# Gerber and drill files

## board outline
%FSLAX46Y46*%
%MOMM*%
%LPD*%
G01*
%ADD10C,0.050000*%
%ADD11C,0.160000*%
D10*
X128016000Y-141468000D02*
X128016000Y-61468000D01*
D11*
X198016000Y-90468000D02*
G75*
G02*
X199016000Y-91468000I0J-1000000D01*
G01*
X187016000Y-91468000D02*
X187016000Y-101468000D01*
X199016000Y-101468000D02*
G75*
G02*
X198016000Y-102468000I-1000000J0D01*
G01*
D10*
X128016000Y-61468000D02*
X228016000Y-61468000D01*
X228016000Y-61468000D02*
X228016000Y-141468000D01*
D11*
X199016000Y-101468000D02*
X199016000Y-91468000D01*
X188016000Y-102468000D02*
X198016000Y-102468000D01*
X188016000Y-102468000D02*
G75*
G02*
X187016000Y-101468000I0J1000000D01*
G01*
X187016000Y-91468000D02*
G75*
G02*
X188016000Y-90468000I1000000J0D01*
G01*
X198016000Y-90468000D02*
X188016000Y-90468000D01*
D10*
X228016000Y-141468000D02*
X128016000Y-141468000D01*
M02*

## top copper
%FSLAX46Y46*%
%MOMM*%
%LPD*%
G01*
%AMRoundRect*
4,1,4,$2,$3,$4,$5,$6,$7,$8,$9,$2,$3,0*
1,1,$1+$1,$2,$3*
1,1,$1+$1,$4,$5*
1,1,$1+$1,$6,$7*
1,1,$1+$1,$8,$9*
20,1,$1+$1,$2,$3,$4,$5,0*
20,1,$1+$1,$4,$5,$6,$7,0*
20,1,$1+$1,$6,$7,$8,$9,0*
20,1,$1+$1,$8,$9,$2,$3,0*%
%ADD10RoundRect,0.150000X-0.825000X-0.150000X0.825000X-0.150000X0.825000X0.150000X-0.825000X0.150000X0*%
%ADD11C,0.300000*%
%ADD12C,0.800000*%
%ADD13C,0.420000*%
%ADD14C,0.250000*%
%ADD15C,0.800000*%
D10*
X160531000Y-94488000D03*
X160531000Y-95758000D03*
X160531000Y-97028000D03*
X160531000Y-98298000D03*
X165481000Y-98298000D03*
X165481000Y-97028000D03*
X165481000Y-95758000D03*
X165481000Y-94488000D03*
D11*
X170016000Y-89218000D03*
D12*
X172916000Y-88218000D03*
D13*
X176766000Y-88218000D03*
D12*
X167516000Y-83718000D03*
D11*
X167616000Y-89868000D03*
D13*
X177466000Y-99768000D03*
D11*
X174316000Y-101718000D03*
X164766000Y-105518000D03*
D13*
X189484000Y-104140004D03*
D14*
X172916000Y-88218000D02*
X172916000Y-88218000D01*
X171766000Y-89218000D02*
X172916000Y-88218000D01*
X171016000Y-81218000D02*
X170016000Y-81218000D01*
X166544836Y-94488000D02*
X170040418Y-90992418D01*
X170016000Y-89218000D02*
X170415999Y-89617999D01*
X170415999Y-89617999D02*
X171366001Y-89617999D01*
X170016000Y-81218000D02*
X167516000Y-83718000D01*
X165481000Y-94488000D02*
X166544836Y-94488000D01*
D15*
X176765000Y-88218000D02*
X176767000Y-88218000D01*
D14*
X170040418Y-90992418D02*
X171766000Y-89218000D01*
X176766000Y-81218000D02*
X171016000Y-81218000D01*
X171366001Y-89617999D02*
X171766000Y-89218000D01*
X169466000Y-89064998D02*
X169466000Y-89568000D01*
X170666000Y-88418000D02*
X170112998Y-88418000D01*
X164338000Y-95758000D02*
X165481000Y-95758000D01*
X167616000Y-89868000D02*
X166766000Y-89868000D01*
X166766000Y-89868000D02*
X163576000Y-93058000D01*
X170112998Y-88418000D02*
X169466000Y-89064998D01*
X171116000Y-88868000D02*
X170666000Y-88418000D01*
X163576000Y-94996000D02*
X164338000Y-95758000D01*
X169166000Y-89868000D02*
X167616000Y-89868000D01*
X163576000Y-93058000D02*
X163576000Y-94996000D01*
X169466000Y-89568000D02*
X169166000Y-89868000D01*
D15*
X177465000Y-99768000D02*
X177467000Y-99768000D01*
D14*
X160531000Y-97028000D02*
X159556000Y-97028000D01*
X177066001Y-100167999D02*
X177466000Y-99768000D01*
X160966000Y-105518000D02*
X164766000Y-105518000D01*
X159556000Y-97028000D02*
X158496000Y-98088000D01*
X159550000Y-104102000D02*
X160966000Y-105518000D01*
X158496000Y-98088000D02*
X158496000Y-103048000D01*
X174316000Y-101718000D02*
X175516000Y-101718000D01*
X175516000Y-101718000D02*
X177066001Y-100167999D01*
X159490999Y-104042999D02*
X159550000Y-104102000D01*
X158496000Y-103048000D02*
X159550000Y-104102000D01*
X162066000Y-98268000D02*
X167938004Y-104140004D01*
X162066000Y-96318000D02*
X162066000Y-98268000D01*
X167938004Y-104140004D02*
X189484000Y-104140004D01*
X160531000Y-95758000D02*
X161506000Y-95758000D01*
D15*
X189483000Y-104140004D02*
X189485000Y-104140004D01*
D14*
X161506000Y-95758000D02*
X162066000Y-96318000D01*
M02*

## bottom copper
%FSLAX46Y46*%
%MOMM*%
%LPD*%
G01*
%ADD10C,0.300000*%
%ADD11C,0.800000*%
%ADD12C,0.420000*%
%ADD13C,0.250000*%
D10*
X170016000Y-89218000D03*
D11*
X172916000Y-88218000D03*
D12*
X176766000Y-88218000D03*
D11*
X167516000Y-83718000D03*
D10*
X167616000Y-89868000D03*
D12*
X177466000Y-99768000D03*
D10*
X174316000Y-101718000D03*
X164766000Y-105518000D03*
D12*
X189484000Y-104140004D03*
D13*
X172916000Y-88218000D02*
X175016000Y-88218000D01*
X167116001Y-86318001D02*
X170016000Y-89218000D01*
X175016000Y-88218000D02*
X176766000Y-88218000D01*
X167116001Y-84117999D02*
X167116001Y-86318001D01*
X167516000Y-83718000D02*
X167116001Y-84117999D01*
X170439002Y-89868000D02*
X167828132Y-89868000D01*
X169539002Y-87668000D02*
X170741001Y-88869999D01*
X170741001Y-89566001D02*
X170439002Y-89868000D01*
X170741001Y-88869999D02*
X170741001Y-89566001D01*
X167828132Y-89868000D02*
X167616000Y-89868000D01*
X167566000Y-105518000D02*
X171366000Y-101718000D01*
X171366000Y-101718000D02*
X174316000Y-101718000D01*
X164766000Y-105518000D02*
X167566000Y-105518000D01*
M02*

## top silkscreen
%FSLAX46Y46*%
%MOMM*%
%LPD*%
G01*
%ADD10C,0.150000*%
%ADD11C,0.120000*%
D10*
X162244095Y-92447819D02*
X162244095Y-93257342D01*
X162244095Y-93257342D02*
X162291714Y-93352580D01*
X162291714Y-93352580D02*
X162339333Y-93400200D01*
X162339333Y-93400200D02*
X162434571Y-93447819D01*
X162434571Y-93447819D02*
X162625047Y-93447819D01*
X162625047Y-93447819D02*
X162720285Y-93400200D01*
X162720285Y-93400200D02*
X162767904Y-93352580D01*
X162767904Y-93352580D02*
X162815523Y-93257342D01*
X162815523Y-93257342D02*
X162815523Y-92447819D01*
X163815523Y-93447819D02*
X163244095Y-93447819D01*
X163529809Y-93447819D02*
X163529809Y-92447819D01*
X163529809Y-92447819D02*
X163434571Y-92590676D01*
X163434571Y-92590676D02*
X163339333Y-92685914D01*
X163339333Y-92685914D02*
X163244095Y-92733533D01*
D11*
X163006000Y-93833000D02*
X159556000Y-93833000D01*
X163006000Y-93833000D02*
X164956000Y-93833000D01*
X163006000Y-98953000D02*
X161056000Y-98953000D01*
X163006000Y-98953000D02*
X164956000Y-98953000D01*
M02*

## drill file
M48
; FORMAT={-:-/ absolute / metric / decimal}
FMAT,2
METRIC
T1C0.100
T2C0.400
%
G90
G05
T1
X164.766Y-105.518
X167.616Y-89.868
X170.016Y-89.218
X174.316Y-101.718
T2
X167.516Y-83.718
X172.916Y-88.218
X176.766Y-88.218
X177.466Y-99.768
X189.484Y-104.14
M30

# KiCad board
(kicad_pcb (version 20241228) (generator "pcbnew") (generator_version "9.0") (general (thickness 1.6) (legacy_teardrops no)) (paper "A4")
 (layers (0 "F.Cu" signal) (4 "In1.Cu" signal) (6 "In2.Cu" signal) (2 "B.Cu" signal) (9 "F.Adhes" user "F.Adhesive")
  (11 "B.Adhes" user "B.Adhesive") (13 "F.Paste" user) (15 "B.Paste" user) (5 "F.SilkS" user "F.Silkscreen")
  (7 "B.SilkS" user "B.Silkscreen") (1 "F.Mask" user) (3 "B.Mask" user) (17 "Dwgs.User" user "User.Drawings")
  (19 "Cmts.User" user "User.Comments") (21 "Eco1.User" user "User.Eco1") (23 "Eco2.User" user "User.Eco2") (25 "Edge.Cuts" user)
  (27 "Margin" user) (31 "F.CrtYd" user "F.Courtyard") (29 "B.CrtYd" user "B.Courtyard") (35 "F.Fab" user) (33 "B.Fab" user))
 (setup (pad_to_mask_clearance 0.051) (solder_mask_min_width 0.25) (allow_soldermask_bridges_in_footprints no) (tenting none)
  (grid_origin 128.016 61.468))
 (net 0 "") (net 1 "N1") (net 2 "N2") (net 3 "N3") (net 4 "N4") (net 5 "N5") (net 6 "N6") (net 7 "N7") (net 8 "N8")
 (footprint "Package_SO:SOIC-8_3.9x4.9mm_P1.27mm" (layer "F.Cu") (at 163.006 96.393)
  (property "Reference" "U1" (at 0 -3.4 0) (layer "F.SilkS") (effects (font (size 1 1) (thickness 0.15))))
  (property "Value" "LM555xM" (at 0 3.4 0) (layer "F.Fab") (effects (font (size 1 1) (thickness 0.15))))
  (fp_line (start 0 -2.56) (end -3.45 -2.56) (stroke (width 0.12) (type solid)) (layer "F.SilkS"))
  (fp_line (start 0 -2.56) (end 1.95 -2.56) (stroke (width 0.12) (type solid)) (layer "F.SilkS"))
  (fp_line (start 0 2.56) (end -1.95 2.56) (stroke (width 0.12) (type solid)) (layer "F.SilkS"))
  (fp_line (start 0 2.56) (end 1.95 2.56) (stroke (width 0.12) (type solid)) (layer "F.SilkS"))
  (pad "1" smd roundrect (at -2.475 -1.905) (size 1.95 0.6) (layers "F.Cu" "F.Mask" "F.Paste") (roundrect_rratio 0.25) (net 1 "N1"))
  (pad "2" smd roundrect (at -2.475 -0.635) (size 1.95 0.6) (layers "F.Cu" "F.Mask" "F.Paste") (roundrect_rratio 0.25) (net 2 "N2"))
  (pad "3" smd roundrect (at -2.475 0.635) (size 1.95 0.6) (layers "F.Cu" "F.Mask" "F.Paste") (roundrect_rratio 0.25) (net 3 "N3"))
  (pad "4" smd roundrect (at -2.475 1.905) (size 1.95 0.6) (layers "F.Cu" "F.Mask" "F.Paste") (roundrect_rratio 0.25) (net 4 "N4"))
  (pad "5" smd roundrect (at 2.475 1.905) (size 1.95 0.6) (layers "F.Cu" "F.Mask" "F.Paste") (roundrect_rratio 0.25) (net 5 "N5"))
  (pad "6" smd roundrect (at 2.475 0.635) (size 1.95 0.6) (layers "F.Cu" "F.Mask" "F.Paste") (roundrect_rratio 0.25) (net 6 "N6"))
  (pad "7" smd roundrect (at 2.475 -0.635) (size 1.95 0.6) (layers "F.Cu" "F.Mask" "F.Paste") (roundrect_rratio 0.25) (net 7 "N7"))
  (pad "8" smd roundrect (at 2.475 -1.905) (size 1.95 0.6) (layers "F.Cu" "F.Mask" "F.Paste") (roundrect_rratio 0.25) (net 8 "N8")))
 (gr_line (start 128.016 141.468) (end 128.016 61.468) (stroke (width 0.05) (type solid)) (layer "Edge.Cuts"))
 (gr_arc (start 198.016 90.468) (mid 198.723107 90.760893) (end 199.016 91.468) (stroke (width 0.16) (type solid)) (layer "Edge.Cuts"))
 (gr_line (start 187.016 91.468) (end 187.016 101.468) (stroke (width 0.16) (type solid)) (layer "Edge.Cuts"))
 (gr_arc (start 199.016 101.468) (mid 198.723107 102.175107) (end 198.016 102.468) (stroke (width 0.16) (type solid)) (layer "Edge.Cuts"))
 (gr_line (start 128.016 61.468) (end 228.016 61.468) (stroke (width 0.05) (type solid)) (layer "Edge.Cuts"))
 (gr_line (start 228.016 61.468) (end 228.016 141.468) (stroke (width 0.05) (type solid)) (layer "Edge.Cuts"))
 (gr_line (start 199.016 101.468) (end 199.016 91.468) (stroke (width 0.16) (type solid)) (layer "Edge.Cuts"))
 (gr_line (start 188.016 102.468) (end 198.016 102.468) (stroke (width 0.16) (type solid)) (layer "Edge.Cuts"))
 (gr_arc (start 188.016 102.468) (mid 187.308893 102.175107) (end 187.016 101.468) (stroke (width 0.16) (type solid)) (layer "Edge.Cuts"))
 (gr_arc (start 187.016 91.468) (mid 187.308893 90.760893) (end 188.016 90.468) (stroke (width 0.16) (type solid)) (layer "Edge.Cuts"))
 (gr_line (start 198.016 90.468) (end 188.016 90.468) (stroke (width 0.16) (type solid)) (layer "Edge.Cuts"))
 (gr_line (start 228.016 141.468) (end 128.016 141.468) (stroke (width 0.05) (type solid)) (layer "Edge.Cuts"))
 (segment (start 172.916 88.218) (end 172.916 88.218) (width 0.25) (layer "F.Cu") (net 8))
 (segment (start 171.766 89.218) (end 172.916 88.218) (width 0.25) (layer "F.Cu") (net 8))
 (segment (start 171.016 81.218) (end 170.016 81.218) (width 0.25) (layer "F.Cu") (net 8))
 (segment (start 166.544836 94.488) (end 170.040418 90.992418) (width 0.25) (layer "F.Cu") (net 8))
 (segment (start 170.016 89.218) (end 170.415999 89.617999) (width 0.25) (layer "F.Cu") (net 8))
 (segment (start 170.415999 89.617999) (end 171.366001 89.617999) (width 0.25) (layer "F.Cu") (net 8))
 (segment (start 170.016 81.218) (end 167.516 83.718) (width 0.25) (layer "F.Cu") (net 8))
 (segment (start 165.481 94.488) (end 166.544836 94.488) (width 0.25) (layer "F.Cu") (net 8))
 (segment (start 176.765 88.218) (end 176.767 88.218) (width 0.8) (layer "F.Cu") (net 8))
 (segment (start 170.040418 90.992418) (end 171.766 89.218) (width 0.25) (layer "F.Cu") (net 8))
 (segment (start 176.766 81.218) (end 171.016 81.218) (width 0.25) (layer "F.Cu") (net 8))
 (segment (start 171.366001 89.617999) (end 171.766 89.218) (width 0.25) (layer "F.Cu") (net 8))
 (via (at 170.016 89.218) (size 0.3) (drill 0.1) (layers "F.Cu" "B.Cu") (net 8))
 (via (at 172.916 88.218) (size 0.8) (drill 0.4) (layers "F.Cu" "B.Cu") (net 8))
 (via (at 176.766 88.218) (size 0.42) (drill 0.4) (layers "F.Cu" "B.Cu") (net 8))
 (via (at 167.516 83.718) (size 0.8) (drill 0.4) (layers "F.Cu" "B.Cu") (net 8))
 (segment (start 172.916 88.218) (end 175.016 88.218) (width 0.25) (layer "B.Cu") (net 8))
 (segment (start 167.116001 86.318001) (end 170.016 89.218) (width 0.25) (layer "B.Cu") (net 8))
 (segment (start 175.016 88.218) (end 176.766 88.218) (width 0.25) (layer "B.Cu") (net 8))
 (segment (start 167.116001 84.117999) (end 167.116001 86.318001) (width 0.25) (layer "B.Cu") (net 8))
 (segment (start 167.516 83.718) (end 167.116001 84.117999) (width 0.25) (layer "B.Cu") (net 8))
 (segment (start 169.466 89.064998) (end 169.466 89.568) (width 0.25) (layer "F.Cu") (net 7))
 (segment (start 170.666 88.418) (end 170.112998 88.418) (width 0.25) (layer "F.Cu") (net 7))
 (segment (start 164.338 95.758) (end 165.481 95.758) (width 0.25) (layer "F.Cu") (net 7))
 (segment (start 167.616 89.868) (end 166.766 89.868) (width 0.25) (layer "F.Cu") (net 7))
 (segment (start 166.766 89.868) (end 163.576 93.058) (width 0.25) (layer "F.Cu") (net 7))
 (segment (start 170.112998 88.418) (end 169.466 89.064998) (width 0.25) (layer "F.Cu") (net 7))
 (segment (start 171.116 88.868) (end 170.666 88.418) (width 0.25) (layer "F.Cu") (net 7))
 (segment (start 163.576 94.996) (end 164.338 95.758) (width 0.25) (layer "F.Cu") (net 7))
 (segment (start 169.166 89.868) (end 167.616 89.868) (width 0.25) (layer "F.Cu") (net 7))
 (segment (start 163.576 93.058) (end 163.576 94.996) (width 0.25) (layer "F.Cu") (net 7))
 (segment (start 169.466 89.568) (end 169.166 89.868) (width 0.25) (layer "F.Cu") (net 7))
 (via (at 167.616 89.868) (size 0.3) (drill 0.1) (layers "F.Cu" "B.Cu") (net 7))
 (segment (start 170.439002 89.868) (end 167.828132 89.868) (width 0.25) (layer "B.Cu") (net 7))
 (segment (start 169.539002 87.668) (end 170.741001 88.869999) (width 0.25) (layer "B.Cu") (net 7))
 (segment (start 170.741001 89.566001) (end 170.439002 89.868) (width 0.25) (layer "B.Cu") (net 7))
 (segment (start 170.741001 88.869999) (end 170.741001 89.566001) (width 0.25) (layer "B.Cu") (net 7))
 (segment (start 167.828132 89.868) (end 167.616 89.868) (width 0.25) (layer "B.Cu") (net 7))
 (segment (start 177.465 99.768) (end 177.467 99.768) (width 0.8) (layer "F.Cu") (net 3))
 (segment (start 160.531 97.028) (end 159.556 97.028) (width 0.25) (layer "F.Cu") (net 3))
 (segment (start 177.066001 100.167999) (end 177.466 99.768) (width 0.25) (layer "F.Cu") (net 3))
 (segment (start 160.966 105.518) (end 164.766 105.518) (width 0.25) (layer "F.Cu") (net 3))
 (segment (start 159.556 97.028) (end 158.496 98.088) (width 0.25) (layer "F.Cu") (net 3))
 (segment (start 159.55 104.102) (end 160.966 105.518) (width 0.25) (layer "F.Cu") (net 3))
 (segment (start 158.496 98.088) (end 158.496 103.048) (width 0.25) (layer "F.Cu") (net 3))
 (segment (start 174.316 101.718) (end 175.516 101.718) (width 0.25) (layer "F.Cu") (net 3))
 (segment (start 175.516 101.718) (end 177.066001 100.167999) (width 0.25) (layer "F.Cu") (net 3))
 (segment (start 159.490999 104.042999) (end 159.55 104.102) (width 0.25) (layer "F.Cu") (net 3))
 (segment (start 158.496 103.048) (end 159.55 104.102) (width 0.25) (layer "F.Cu") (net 3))
 (via (at 177.466 99.768) (size 0.42) (drill 0.4) (layers "F.Cu" "B.Cu") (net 3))
 (via (at 174.316 101.718) (size 0.3) (drill 0.1) (layers "F.Cu" "B.Cu") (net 3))
 (via (at 164.766 105.518) (size 0.3) (drill 0.1) (layers "F.Cu" "B.Cu") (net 3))
 (segment (start 167.566 105.518) (end 171.366 101.718) (width 0.25) (layer "B.Cu") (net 3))
 (segment (start 171.366 101.718) (end 174.316 101.718) (width 0.25) (layer "B.Cu") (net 3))
 (segment (start 164.766 105.518) (end 167.566 105.518) (width 0.25) (layer "B.Cu") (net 3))
 (segment (start 162.066 98.268) (end 167.938004 104.140004) (width 0.25) (layer "F.Cu") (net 2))
 (segment (start 162.066 96.318) (end 162.066 98.268) (width 0.25) (layer "F.Cu") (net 2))
 (segment (start 167.938004 104.140004) (end 189.484 104.140004) (width 0.25) (layer "F.Cu") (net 2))
 (segment (start 160.531 95.758) (end 161.506 95.758) (width 0.25) (layer "F.Cu") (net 2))
 (segment (start 189.483 104.140004) (end 189.485 104.140004) (width 0.8) (layer "F.Cu") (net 2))
 (segment (start 161.506 95.758) (end 162.066 96.318) (width 0.25) (layer "F.Cu") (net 2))
 (via (at 189.484 104.140004) (size 0.42) (drill 0.4) (layers "F.Cu" "B.Cu") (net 2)))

